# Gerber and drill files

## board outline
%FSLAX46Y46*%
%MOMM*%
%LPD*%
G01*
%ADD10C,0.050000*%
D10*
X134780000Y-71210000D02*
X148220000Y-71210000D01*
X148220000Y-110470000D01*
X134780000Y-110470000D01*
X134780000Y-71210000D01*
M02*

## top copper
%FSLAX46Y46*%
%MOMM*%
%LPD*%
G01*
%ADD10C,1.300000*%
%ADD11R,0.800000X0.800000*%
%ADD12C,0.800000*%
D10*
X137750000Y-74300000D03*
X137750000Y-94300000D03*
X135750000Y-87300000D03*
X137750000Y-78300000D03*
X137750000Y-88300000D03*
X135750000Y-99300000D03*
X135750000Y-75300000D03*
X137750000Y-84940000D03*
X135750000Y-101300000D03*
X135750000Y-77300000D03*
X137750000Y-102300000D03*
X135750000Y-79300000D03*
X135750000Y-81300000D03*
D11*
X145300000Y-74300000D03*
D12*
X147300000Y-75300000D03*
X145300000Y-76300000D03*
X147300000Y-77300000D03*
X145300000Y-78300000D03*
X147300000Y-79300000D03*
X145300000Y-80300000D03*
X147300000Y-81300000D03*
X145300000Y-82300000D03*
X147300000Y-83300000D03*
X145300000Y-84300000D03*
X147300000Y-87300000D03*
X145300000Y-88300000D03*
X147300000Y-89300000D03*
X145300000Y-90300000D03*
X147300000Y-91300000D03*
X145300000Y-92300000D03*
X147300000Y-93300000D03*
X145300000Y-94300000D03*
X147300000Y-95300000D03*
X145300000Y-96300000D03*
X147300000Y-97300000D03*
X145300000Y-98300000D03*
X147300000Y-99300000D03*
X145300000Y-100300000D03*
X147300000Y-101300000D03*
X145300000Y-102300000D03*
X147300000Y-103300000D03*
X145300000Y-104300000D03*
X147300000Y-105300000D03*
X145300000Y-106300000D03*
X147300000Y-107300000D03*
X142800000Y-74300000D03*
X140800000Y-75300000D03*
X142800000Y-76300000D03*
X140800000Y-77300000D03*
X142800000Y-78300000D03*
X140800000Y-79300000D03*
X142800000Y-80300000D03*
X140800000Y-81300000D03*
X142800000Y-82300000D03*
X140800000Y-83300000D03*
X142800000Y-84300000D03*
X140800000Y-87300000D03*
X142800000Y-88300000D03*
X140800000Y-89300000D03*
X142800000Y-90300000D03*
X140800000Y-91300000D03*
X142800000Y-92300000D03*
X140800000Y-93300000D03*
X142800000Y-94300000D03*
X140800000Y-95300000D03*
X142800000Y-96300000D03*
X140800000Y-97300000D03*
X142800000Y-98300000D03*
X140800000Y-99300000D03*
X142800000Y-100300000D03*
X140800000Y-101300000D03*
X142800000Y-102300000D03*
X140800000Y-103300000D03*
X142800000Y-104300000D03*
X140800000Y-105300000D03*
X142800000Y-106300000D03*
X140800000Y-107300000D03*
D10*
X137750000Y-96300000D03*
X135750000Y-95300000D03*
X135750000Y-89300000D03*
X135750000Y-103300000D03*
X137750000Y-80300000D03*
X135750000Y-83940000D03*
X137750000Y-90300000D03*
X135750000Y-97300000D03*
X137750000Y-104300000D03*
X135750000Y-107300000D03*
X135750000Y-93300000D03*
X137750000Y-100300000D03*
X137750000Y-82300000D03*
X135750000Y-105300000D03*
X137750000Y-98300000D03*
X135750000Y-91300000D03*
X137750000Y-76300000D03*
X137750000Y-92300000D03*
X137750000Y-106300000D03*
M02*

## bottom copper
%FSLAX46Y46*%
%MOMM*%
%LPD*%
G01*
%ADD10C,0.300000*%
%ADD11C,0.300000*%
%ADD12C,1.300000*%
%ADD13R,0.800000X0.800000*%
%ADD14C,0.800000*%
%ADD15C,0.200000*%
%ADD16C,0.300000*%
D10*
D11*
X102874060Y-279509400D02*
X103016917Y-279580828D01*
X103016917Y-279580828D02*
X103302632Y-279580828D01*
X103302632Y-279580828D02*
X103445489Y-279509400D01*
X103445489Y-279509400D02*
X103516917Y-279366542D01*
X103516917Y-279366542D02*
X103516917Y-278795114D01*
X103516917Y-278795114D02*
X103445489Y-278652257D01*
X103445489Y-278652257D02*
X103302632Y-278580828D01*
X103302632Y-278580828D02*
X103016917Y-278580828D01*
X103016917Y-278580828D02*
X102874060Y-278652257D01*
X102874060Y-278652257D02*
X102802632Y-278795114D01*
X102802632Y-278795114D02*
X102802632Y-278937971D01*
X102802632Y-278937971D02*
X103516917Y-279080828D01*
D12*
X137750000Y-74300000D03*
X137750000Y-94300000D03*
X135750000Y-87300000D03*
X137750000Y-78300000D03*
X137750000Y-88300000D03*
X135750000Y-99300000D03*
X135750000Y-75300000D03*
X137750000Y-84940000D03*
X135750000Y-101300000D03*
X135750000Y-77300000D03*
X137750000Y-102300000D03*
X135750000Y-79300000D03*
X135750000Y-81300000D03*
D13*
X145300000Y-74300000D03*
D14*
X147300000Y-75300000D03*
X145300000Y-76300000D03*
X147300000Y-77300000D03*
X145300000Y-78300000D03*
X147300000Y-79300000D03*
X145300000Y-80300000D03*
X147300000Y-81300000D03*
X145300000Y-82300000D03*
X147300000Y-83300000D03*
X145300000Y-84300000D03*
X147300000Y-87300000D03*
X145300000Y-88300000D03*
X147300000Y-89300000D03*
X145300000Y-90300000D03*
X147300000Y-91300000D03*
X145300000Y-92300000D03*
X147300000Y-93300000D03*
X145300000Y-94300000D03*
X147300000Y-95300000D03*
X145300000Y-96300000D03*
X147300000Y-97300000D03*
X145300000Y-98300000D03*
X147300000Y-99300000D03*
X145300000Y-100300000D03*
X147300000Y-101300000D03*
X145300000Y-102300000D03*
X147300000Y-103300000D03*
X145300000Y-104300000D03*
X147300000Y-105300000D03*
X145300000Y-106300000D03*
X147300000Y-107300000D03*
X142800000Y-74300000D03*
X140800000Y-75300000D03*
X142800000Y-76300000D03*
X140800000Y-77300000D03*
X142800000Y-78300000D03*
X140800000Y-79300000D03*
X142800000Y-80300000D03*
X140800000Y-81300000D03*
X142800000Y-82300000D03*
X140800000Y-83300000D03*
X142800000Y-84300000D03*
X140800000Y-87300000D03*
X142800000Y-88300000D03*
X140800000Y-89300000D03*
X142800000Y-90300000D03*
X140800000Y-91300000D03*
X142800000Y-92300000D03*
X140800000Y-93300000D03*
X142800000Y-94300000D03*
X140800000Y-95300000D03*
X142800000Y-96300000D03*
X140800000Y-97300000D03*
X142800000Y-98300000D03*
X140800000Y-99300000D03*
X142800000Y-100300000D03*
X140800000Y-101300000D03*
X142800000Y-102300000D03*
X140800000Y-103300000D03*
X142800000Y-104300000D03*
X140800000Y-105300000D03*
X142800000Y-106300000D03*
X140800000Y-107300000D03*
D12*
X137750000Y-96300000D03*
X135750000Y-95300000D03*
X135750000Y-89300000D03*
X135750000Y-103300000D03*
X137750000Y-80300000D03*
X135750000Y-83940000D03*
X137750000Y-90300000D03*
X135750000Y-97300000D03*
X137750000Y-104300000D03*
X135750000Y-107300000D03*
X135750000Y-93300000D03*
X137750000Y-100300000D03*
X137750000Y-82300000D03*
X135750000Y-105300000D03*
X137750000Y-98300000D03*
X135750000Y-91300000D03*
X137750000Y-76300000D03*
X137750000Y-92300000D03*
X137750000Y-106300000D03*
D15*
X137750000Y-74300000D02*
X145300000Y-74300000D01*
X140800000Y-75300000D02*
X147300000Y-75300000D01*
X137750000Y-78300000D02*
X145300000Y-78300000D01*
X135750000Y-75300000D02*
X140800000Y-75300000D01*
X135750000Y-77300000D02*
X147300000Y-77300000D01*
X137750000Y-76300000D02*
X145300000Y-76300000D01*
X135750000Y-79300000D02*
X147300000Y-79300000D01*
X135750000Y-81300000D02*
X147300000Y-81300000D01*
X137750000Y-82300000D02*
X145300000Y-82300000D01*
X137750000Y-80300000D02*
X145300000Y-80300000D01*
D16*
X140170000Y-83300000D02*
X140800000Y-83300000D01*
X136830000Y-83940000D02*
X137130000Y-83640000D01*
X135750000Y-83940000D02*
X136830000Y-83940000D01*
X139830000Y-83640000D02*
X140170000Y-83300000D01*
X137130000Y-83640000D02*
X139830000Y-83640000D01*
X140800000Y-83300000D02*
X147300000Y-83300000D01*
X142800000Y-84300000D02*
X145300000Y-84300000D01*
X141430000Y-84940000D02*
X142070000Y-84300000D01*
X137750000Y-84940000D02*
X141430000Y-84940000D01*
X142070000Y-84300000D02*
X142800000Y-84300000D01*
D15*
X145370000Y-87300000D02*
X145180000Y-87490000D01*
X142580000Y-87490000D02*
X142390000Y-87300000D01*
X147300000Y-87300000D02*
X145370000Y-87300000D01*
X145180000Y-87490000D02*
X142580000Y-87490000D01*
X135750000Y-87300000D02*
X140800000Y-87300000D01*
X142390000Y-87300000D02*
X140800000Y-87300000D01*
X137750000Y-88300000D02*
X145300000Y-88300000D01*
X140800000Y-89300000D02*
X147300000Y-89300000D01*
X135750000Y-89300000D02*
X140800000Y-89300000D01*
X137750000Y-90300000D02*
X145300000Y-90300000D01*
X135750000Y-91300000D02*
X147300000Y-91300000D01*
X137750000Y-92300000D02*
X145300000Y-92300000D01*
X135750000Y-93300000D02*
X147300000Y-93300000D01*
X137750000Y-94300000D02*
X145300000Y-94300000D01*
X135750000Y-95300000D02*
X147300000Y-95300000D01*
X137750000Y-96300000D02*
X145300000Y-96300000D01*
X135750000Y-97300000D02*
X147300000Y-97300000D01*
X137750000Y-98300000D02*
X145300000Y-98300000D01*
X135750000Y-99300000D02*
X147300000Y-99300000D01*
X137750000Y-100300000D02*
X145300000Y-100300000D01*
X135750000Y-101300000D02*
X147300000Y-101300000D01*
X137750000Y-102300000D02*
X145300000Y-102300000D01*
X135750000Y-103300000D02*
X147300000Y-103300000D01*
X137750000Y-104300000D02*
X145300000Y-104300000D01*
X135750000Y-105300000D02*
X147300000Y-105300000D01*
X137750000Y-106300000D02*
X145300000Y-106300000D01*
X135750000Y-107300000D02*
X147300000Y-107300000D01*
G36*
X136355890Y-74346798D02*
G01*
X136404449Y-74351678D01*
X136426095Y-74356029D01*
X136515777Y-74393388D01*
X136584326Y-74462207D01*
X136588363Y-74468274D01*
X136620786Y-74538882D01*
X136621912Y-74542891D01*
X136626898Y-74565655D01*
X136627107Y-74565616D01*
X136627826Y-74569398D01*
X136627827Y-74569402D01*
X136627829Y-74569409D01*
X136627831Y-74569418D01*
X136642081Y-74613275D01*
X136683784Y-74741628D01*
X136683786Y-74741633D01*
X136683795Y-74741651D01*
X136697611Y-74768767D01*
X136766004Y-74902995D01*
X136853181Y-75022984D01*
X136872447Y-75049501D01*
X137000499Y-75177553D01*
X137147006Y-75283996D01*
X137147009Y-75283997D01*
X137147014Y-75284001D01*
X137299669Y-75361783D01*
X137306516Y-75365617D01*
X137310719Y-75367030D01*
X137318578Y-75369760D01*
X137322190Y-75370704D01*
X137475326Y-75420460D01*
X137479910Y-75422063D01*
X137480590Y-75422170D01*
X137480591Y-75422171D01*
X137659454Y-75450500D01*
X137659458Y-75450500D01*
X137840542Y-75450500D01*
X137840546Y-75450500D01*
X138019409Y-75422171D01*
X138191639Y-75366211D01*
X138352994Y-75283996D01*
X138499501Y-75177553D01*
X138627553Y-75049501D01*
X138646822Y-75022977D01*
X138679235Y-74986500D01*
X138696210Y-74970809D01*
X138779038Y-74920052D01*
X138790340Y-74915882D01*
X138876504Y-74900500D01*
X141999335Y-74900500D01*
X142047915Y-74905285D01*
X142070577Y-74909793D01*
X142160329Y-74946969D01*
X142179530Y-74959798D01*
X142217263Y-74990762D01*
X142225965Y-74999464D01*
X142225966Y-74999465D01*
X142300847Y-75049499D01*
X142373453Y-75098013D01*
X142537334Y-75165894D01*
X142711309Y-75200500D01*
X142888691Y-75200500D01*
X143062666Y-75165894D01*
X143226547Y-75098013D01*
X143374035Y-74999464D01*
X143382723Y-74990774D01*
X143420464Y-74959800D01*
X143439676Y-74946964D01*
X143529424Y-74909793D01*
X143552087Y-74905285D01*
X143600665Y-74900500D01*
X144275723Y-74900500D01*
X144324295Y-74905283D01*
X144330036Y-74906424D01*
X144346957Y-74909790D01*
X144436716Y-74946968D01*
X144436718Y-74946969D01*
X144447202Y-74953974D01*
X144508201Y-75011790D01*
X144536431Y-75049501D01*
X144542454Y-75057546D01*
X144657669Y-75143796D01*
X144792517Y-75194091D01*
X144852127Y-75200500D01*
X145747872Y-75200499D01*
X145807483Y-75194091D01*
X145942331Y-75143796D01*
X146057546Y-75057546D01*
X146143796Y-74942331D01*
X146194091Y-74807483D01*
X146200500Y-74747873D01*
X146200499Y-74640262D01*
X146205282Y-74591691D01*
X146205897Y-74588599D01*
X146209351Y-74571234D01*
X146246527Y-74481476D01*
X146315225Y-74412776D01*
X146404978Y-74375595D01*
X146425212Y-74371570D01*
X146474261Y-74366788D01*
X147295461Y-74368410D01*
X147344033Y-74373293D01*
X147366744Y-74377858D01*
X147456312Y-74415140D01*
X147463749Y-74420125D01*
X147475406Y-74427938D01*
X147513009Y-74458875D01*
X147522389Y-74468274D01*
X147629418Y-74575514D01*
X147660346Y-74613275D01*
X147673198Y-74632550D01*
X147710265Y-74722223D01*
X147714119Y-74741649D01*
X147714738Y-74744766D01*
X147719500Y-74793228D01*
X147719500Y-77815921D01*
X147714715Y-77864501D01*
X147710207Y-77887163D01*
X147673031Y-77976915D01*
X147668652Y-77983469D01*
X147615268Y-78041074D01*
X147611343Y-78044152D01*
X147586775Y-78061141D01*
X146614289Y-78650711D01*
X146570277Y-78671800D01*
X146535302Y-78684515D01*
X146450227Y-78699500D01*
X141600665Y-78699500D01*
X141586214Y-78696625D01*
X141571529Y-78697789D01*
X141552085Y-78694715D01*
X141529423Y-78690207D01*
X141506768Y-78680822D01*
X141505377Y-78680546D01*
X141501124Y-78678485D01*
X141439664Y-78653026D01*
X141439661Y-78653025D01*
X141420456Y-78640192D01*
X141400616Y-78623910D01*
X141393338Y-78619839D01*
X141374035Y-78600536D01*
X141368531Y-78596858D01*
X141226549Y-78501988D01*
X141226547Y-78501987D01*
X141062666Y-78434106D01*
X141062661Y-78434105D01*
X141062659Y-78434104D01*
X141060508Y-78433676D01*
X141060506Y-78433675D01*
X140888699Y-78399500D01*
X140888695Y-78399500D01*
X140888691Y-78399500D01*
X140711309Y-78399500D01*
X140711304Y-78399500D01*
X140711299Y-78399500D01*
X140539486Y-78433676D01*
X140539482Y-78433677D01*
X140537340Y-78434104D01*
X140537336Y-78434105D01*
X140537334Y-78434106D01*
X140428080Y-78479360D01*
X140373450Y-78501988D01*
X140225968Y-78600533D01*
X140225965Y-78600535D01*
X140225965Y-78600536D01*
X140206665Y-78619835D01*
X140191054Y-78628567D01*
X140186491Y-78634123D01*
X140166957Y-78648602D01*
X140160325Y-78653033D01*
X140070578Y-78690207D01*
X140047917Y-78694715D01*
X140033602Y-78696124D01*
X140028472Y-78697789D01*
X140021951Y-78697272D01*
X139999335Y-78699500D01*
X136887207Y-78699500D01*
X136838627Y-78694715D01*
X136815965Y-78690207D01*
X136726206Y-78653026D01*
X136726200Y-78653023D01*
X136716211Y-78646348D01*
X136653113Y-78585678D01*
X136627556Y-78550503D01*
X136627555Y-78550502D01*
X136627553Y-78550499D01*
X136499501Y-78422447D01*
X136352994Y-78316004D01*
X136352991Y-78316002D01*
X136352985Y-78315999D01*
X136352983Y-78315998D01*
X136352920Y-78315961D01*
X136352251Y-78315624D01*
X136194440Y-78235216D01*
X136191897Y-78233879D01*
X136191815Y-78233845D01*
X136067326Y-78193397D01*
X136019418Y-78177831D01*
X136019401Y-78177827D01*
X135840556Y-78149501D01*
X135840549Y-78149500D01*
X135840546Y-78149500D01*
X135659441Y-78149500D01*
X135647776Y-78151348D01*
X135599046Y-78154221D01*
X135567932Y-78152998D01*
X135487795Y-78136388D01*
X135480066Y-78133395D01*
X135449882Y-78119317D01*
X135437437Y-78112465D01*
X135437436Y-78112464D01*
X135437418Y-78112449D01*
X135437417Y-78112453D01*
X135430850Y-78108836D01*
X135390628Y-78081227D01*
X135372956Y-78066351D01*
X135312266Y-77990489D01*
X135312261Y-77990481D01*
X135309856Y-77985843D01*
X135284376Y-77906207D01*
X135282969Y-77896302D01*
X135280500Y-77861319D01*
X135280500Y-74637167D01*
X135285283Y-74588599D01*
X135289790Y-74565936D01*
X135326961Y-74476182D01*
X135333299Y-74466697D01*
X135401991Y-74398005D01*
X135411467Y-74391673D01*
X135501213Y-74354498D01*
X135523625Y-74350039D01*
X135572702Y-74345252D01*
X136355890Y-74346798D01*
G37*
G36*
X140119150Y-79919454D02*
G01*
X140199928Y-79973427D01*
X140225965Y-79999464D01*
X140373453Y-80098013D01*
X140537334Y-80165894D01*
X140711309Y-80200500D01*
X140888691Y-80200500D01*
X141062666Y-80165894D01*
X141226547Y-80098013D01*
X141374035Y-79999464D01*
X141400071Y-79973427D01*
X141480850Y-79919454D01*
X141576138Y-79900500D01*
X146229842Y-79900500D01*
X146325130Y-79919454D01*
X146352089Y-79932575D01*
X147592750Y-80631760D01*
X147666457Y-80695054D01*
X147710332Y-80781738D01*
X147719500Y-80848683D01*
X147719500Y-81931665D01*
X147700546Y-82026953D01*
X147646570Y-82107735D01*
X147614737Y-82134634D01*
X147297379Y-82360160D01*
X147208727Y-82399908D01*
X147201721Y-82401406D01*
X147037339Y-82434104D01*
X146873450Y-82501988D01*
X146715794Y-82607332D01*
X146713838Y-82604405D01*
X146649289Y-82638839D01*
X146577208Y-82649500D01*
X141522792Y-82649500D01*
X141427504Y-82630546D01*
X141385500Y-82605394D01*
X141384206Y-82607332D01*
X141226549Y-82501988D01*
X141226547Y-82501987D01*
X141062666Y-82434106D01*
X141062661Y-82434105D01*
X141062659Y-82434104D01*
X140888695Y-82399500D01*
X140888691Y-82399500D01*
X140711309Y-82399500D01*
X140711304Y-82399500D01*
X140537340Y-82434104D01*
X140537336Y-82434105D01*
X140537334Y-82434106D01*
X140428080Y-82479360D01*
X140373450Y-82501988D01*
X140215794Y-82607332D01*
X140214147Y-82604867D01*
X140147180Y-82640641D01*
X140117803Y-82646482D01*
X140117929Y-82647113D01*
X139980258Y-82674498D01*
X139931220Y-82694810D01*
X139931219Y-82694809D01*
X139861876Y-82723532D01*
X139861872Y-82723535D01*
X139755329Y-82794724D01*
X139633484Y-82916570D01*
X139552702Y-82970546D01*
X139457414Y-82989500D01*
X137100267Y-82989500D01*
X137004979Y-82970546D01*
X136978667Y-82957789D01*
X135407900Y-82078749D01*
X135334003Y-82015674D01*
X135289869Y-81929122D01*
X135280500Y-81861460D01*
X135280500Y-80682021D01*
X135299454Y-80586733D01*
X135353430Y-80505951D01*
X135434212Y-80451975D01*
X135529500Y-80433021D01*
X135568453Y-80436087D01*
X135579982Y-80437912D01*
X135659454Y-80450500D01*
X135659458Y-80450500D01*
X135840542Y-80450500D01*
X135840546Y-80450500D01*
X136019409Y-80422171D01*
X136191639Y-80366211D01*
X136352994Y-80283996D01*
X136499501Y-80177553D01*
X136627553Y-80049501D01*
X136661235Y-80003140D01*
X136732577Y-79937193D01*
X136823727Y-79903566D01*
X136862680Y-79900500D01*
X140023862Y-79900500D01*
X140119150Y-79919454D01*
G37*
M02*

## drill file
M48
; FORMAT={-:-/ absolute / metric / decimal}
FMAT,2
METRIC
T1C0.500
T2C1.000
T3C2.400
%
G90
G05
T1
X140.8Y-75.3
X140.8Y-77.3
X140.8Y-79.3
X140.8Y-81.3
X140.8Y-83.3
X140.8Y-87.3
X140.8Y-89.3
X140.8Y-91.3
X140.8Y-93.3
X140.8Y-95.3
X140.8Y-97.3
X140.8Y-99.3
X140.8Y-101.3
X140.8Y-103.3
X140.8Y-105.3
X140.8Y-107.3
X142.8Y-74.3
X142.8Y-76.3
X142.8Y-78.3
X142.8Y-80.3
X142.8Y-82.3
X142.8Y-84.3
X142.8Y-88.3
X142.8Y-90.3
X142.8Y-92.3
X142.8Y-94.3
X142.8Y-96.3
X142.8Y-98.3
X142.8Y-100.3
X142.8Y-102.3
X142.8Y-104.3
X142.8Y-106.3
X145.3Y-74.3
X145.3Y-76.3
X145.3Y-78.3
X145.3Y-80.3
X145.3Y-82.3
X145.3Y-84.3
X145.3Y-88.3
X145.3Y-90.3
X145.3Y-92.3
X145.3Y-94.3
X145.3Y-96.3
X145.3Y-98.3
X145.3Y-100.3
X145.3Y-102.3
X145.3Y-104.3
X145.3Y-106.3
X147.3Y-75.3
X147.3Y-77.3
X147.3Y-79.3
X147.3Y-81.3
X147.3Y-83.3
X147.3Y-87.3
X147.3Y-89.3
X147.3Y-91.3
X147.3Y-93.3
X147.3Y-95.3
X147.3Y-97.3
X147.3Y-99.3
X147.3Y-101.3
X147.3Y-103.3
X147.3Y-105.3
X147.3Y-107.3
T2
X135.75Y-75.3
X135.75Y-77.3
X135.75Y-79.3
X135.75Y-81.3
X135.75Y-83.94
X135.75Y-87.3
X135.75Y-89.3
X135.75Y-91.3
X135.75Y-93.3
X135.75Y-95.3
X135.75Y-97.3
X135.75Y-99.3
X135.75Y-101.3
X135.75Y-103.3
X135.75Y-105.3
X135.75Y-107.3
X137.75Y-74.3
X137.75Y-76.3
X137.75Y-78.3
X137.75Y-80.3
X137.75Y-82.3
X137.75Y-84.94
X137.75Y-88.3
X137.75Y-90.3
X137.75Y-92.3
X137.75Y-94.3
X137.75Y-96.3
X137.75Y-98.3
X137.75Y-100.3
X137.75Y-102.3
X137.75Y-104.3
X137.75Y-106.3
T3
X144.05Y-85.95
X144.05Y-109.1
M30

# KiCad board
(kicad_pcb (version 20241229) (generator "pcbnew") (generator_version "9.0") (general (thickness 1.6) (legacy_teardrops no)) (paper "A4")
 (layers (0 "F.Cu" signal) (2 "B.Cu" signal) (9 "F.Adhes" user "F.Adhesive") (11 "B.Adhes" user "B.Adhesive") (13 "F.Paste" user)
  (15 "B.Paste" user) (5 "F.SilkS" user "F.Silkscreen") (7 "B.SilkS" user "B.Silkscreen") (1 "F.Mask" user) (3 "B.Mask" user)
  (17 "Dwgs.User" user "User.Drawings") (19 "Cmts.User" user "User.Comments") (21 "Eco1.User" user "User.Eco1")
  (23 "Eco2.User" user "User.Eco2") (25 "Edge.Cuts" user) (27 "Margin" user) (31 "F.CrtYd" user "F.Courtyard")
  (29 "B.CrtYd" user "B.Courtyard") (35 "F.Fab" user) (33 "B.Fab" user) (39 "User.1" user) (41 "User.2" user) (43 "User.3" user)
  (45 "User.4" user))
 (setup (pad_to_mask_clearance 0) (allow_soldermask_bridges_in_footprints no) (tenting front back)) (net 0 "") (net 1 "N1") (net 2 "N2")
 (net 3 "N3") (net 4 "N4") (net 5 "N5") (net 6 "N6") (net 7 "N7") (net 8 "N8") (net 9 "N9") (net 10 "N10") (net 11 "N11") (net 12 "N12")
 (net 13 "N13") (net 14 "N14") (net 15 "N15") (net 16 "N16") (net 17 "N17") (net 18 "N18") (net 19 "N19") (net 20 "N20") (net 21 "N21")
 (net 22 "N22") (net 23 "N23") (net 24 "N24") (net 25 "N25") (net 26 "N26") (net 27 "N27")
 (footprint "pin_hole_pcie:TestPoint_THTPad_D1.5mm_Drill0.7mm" (layer "F.Cu") (at 137.75 74.3 180)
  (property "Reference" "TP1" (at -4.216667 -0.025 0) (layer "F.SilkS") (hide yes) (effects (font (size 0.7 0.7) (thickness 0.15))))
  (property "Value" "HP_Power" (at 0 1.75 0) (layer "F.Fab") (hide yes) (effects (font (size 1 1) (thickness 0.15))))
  (pad "1" thru_hole circle (at 0 0 180) (size 1.3 1.3) (drill 1) (layers "*.Cu" "*.Mask") (remove_unused_layers no) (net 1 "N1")))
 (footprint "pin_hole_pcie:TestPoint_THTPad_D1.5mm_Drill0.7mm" (layer "F.Cu") (at 137.75 94.3 180)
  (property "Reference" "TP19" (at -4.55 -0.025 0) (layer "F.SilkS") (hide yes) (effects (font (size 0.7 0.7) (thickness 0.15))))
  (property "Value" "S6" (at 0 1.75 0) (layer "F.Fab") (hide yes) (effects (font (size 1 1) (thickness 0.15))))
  (pad "1" thru_hole circle (at 0 0 180) (size 1.3 1.5) (drill 1) (layers "*.Cu" "*.Mask") (remove_unused_layers no) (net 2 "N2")))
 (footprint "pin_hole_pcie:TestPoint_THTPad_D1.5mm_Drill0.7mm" (layer "F.Cu") (at 135.75 87.3 180)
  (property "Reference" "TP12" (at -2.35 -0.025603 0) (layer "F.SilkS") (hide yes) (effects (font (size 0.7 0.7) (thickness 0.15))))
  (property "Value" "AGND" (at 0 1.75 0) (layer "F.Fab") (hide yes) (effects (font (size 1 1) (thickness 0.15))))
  (pad "1" thru_hole circle (at 0 0 180) (size 1.3 1.5) (drill 1) (layers "*.Cu" "*.Mask") (remove_unused_layers no) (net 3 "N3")))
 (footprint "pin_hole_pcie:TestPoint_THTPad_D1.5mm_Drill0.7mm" (layer "F.Cu") (at 137.75 78.3 180)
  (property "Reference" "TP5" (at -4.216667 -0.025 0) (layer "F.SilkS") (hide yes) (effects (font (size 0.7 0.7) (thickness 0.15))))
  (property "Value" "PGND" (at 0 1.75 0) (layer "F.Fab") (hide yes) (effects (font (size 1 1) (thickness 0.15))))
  (pad "1" thru_hole circle (at 0 0 180) (size 1.3 1.5) (drill 1) (layers "*.Cu" "*.Mask") (remove_unused_layers no) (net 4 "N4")))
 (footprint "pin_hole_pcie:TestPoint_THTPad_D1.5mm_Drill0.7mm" (layer "F.Cu") (at 137.75 88.3 180)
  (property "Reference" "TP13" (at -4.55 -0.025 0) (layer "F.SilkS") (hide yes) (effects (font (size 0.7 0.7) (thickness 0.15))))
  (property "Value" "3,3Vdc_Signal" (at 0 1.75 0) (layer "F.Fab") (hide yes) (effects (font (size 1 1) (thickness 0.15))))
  (pad "1" thru_hole circle (at 0 0 180) (size 1.3 1.5) (drill 1) (layers "*.Cu" "*.Mask") (remove_unused_layers no) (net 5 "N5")))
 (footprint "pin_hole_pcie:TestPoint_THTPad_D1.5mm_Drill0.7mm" (layer "F.Cu") (at 135.75 99.3 180)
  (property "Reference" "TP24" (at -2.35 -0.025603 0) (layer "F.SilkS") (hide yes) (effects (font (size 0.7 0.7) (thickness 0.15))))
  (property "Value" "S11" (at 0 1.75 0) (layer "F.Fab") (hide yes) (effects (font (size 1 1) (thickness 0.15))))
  (pad "1" thru_hole circle (at 0 0 180) (size 1.3 1.5) (drill 1) (layers "*.Cu" "*.Mask") (remove_unused_layers no) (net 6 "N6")))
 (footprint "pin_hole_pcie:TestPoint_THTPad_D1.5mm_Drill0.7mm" (layer "F.Cu") (at 135.75 75.3 180)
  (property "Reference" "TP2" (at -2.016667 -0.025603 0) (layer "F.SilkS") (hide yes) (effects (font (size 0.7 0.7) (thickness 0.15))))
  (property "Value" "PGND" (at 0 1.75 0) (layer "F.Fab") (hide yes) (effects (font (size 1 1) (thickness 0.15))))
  (pad "1" thru_hole circle (at 0 0 180) (size 1.3 1.5) (drill 1) (layers "*.Cu" "*.Mask") (remove_unused_layers no) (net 4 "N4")))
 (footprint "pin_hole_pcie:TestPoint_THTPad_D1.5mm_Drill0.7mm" (layer "F.Cu") (at 137.75 84.94 180)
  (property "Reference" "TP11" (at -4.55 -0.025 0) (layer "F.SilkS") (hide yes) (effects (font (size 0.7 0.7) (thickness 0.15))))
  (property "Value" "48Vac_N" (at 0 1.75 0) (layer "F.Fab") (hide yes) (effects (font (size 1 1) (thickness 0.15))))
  (pad "1" thru_hole circle (at 0 0 180) (size 1.3 1.5) (drill 1) (layers "*.Cu" "*.Mask") (remove_unused_layers no) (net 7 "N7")))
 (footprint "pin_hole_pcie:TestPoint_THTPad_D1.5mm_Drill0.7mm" (layer "F.Cu") (at 135.75 101.3 180)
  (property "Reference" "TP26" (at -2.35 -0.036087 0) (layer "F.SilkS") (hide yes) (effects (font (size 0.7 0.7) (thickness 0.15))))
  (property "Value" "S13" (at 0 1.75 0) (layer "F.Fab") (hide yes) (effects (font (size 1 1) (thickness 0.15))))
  (pad "1" thru_hole circle (at 0 0 180) (size 1.3 1.5) (drill 1) (layers "*.Cu" "*.Mask") (remove_unused_layers no) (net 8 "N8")))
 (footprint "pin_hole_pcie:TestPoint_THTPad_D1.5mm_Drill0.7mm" (layer "F.Cu") (at 135.75 77.3 180)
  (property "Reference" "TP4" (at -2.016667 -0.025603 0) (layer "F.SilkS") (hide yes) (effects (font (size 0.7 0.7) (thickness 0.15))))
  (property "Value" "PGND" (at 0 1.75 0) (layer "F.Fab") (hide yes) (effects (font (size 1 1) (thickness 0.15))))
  (pad "1" thru_hole circle (at 0 0 180) (size 1.3 1.5) (drill 1) (layers "*.Cu" "*.Mask") (remove_unused_layers no) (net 4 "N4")))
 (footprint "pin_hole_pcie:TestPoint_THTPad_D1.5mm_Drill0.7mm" (layer "F.Cu") (at 137.75 102.3 180)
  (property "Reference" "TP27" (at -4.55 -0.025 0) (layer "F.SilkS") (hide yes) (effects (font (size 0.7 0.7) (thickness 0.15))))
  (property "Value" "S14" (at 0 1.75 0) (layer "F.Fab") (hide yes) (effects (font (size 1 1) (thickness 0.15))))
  (pad "1" thru_hole circle (at 0 0 180) (size 1.3 1.5) (drill 1) (layers "*.Cu" "*.Mask") (remove_unused_layers no) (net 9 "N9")))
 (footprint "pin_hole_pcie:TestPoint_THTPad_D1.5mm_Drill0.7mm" (layer "F.Cu") (at 135.75 79.3 180)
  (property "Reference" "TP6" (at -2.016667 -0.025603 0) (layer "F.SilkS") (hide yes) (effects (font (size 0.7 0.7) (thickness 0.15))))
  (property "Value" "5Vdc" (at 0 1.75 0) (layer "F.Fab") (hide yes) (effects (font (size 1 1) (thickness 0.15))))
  (pad "1" thru_hole circle (at 0 0 180) (size 1.3 1.5) (drill 1) (layers "*.Cu" "*.Mask") (remove_unused_layers no) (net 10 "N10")))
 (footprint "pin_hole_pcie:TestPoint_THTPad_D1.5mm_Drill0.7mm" (layer "F.Cu") (at 135.75 81.3 180)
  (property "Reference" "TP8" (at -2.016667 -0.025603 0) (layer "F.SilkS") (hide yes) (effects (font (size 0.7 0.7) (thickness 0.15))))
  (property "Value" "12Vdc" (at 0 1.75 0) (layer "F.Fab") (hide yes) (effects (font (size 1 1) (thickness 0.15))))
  (pad "1" thru_hole circle (at 0 0 180) (size 1.3 1.5) (drill 1) (layers "*.Cu" "*.Mask") (remove_unused_layers no) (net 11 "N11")))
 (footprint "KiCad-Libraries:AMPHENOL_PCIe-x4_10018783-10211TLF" (layer "F.Cu") (at 144.05 85.95 -90)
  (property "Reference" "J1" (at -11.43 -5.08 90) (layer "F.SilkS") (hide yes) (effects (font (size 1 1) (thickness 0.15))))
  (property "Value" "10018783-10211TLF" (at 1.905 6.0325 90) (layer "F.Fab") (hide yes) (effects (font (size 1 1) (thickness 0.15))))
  (pad "" np_thru_hole circle (at 0 0 270) (size 2.4 2.4) (drill 2.4) (layers "*.Cu" "*.Mask"))
  (pad "" np_thru_hole circle (at 23.15 0 270) (size 2.4 2.4) (drill 2.4) (layers "*.Cu" "*.Mask"))
  (pad "A1" thru_hole rect (at -11.65 -1.25 270) (size 0.8 0.8) (drill 0.5) (layers "*.Cu" "*.Mask") (remove_unused_layers no) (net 1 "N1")
   (solder_mask_margin 0.102))
  (pad "A2" thru_hole circle (at -10.65 -3.25 270) (size 0.8 1.288) (drill 0.5) (layers "*.Cu" "*.Mask") (remove_unused_layers no)
   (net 4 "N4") (solder_mask_margin 0.102))
  (pad "A3" thru_hole circle (at -9.65 -1.25 270) (size 0.8 1.288) (drill 0.5) (layers "*.Cu" "*.Mask") (remove_unused_layers no)
   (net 4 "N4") (solder_mask_margin 0.102))
  (pad "A4" thru_hole circle (at -8.65 -3.25 270) (size 0.8 1.288) (drill 0.5) (layers "*.Cu" "*.Mask") (remove_unused_layers no)
   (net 4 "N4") (solder_mask_margin 0.102))
  (pad "A5" thru_hole circle (at -7.65 -1.25 270) (size 0.8 1.288) (drill 0.5) (layers "*.Cu" "*.Mask") (remove_unused_layers no)
   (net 4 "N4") (solder_mask_margin 0.102))
  (pad "A6" thru_hole circle (at -6.65 -3.25 270) (size 0.8 1.288) (drill 0.5) (layers "*.Cu" "*.Mask") (remove_unused_layers no)
   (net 10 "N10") (solder_mask_margin 0.102))
  (pad "A7" thru_hole circle (at -5.65 -1.25 270) (size 0.8 1.288) (drill 0.5) (layers "*.Cu" "*.Mask") (remove_unused_layers no)
   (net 11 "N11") (solder_mask_margin 0.102))
  (pad "A8" thru_hole circle (at -4.65 -3.25 270) (size 0.8 1.288) (drill 0.5) (layers "*.Cu" "*.Mask") (remove_unused_layers no)
   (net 11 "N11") (solder_mask_margin 0.102))
  (pad "A9" thru_hole circle (at -3.65 -1.25 270) (size 0.8 1.288) (drill 0.5) (layers "*.Cu" "*.Mask") (remove_unused_layers no)
   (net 11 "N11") (solder_mask_margin 0.102))
  (pad "A10" thru_hole circle (at -2.65 -3.25 270) (size 0.8 1.288) (drill 0.5) (layers "*.Cu" "*.Mask") (remove_unused_layers no)
   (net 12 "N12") (solder_mask_margin 0.102))
  (pad "A11" thru_hole circle (at -1.65 -1.25 270) (size 0.8 1.288) (drill 0.5) (layers "*.Cu" "*.Mask") (remove_unused_layers no)
   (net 7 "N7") (solder_mask_margin 0.102))
  (pad "A12" thru_hole circle (at 1.35 -3.25 270) (size 0.8 1.288) (drill 0.5) (layers "*.Cu" "*.Mask") (remove_unused_layers no)
   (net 3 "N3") (solder_mask_margin 0.102))
  (pad "A13" thru_hole circle (at 2.35 -1.25 270) (size 0.8 1.288) (drill 0.5) (layers "*.Cu" "*.Mask") (remove_unused_layers no)
   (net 5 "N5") (solder_mask_margin 0.102))
  (pad "A14" thru_hole circle (at 3.35 -3.25 270) (size 0.8 1.288) (drill 0.5) (layers "*.Cu" "*.Mask") (remove_unused_layers no)
   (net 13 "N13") (solder_mask_margin 0.102))
  (pad "A15" thru_hole circle (at 4.35 -1.25 270) (size 0.8 1.288) (drill 0.5) (layers "*.Cu" "*.Mask") (remove_unused_layers no)
   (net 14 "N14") (solder_mask_margin 0.102))
  (pad "A16" thru_hole circle (at 5.35 -3.25 270) (size 0.8 1.288) (drill 0.5) (layers "*.Cu" "*.Mask") (remove_unused_layers no)
   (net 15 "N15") (solder_mask_margin 0.102))
  (pad "A17" thru_hole circle (at 6.35 -1.25 270) (size 0.8 1.288) (drill 0.5) (layers "*.Cu" "*.Mask") (remove_unused_layers no)
   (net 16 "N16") (solder_mask_margin 0.102))
  (pad "A18" thru_hole circle (at 7.35 -3.25 270) (size 0.8 1.288) (drill 0.5) (layers "*.Cu" "*.Mask") (remove_unused_layers no)
   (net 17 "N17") (solder_mask_margin 0.102))
  (pad "A19" thru_hole circle (at 8.35 -1.25 270) (size 0.8 1.288) (drill 0.5) (layers "*.Cu" "*.Mask") (remove_unused_layers no)
   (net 2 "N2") (solder_mask_margin 0.102))
  (pad "A20" thru_hole circle (at 9.35 -3.25 270) (size 0.8 1.288) (drill 0.5) (layers "*.Cu" "*.Mask") (remove_unused_layers no)
   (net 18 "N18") (solder_mask_margin 0.102))
  (pad "A21" thru_hole circle (at 10.35 -1.25 270) (size 0.8 1.288) (drill 0.5) (layers "*.Cu" "*.Mask") (remove_unused_layers no)
   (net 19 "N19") (solder_mask_margin 0.102))
  (pad "A22" thru_hole circle (at 11.35 -3.25 270) (size 0.8 1.288) (drill 0.5) (layers "*.Cu" "*.Mask") (remove_unused_layers no)
   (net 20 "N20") (solder_mask_margin 0.102))
  (pad "A23" thru_hole circle (at 12.35 -1.25 270) (size 0.8 1.288) (drill 0.5) (layers "*.Cu" "*.Mask") (remove_unused_layers no)
   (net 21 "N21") (solder_mask_margin 0.102))
  (pad "A24" thru_hole circle (at 13.35 -3.25 270) (size 0.8 1.288) (drill 0.5) (layers "*.Cu" "*.Mask") (remove_unused_layers no)
   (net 6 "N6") (solder_mask_margin 0.102))
  (pad "A25" thru_hole circle (at 14.35 -1.25 270) (size 0.8 1.288) (drill 0.5) (layers "*.Cu" "*.Mask") (remove_unused_layers no)
   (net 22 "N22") (solder_mask_margin 0.102))
  (pad "A26" thru_hole circle (at 15.35 -3.25 270) (size 0.8 1.288) (drill 0.5) (layers "*.Cu" "*.Mask") (remove_unused_layers no)
   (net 8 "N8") (solder_mask_margin 0.102))
  (pad "A27" thru_hole circle (at 16.35 -1.25 270) (size 0.8 1.288) (drill 0.5) (layers "*.Cu" "*.Mask") (remove_unused_layers no)
   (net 9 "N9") (solder_mask_margin 0.102))
  (pad "A28" thru_hole circle (at 17.35 -3.25 270) (size 0.8 1.288) (drill 0.5) (layers "*.Cu" "*.Mask") (remove_unused_layers no)
   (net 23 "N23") (solder_mask_margin 0.102))
  (pad "A29" thru_hole circle (at 18.35 -1.25 270) (size 0.8 1.288) (drill 0.5) (layers "*.Cu" "*.Mask") (remove_unused_layers no)
   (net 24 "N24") (solder_mask_margin 0.102))
  (pad "A30" thru_hole circle (at 19.35 -3.25 270) (size 0.8 1.288) (drill 0.5) (layers "*.Cu" "*.Mask") (remove_unused_layers no)
   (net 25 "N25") (solder_mask_margin 0.102))
  (pad "A31" thru_hole circle (at 20.35 -1.25 270) (size 0.8 1.288) (drill 0.5) (layers "*.Cu" "*.Mask") (remove_unused_layers no)
   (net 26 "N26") (solder_mask_margin 0.102))
  (pad "A32" thru_hole circle (at 21.35 -3.25 270) (size 0.8 1.288) (drill 0.5) (layers "*.Cu" "*.Mask") (remove_unused_layers no)
   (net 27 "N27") (solder_mask_margin 0.102))
  (pad "B1" thru_hole circle (at -11.65 1.25 270) (size 0.8 1.288) (drill 0.5) (layers "*.Cu" "*.Mask") (remove_unused_layers no)
   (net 1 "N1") (solder_mask_margin 0.102))
  (pad "B2" thru_hole circle (at -10.65 3.25 270) (size 0.8 1.288) (drill 0.5) (layers "*.Cu" "*.Mask") (remove_unused_layers no)
   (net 4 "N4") (solder_mask_margin 0.102))
  (pad "B3" thru_hole circle (at -9.65 1.25 270) (size 0.8 1.288) (drill 0.5) (layers "*.Cu" "*.Mask") (remove_unused_layers no)
   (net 4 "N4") (solder_mask_margin 0.102))
  (pad "B4" thru_hole circle (at -8.65 3.25 270) (size 0.8 1.288) (drill 0.5) (layers "*.Cu" "*.Mask") (remove_unused_layers no)
   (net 4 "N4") (solder_mask_margin 0.102))
  (pad "B5" thru_hole circle (at -7.65 1.25 270) (size 0.8 1.288) (drill 0.5) (layers "*.Cu" "*.Mask") (remove_unused_layers no)
   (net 4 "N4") (solder_mask_margin 0.102))
  (pad "B6" thru_hole circle (at -6.65 3.25 270) (size 0.8 1.288) (drill 0.5) (layers "*.Cu" "*.Mask") (remove_unused_layers no)
   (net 10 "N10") (solder_mask_margin 0.102))
  (pad "B7" thru_hole circle (at -5.65 1.25 270) (size 0.8 1.288) (drill 0.5) (layers "*.Cu" "*.Mask") (remove_unused_layers no)
   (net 11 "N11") (solder_mask_margin 0.102))
  (pad "B8" thru_hole circle (at -4.65 3.25 270) (size 0.8 1.288) (drill 0.5) (layers "*.Cu" "*.Mask") (remove_unused_layers no)
   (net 11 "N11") (solder_mask_margin 0.102))
  (pad "B9" thru_hole circle (at -3.65 1.25 270) (size 0.8 1.288) (drill 0.5) (layers "*.Cu" "*.Mask") (remove_unused_layers no)
   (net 11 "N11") (solder_mask_margin 0.102))
  (pad "B10" thru_hole circle (at -2.65 3.25 270) (size 0.8 1.288) (drill 0.5) (layers "*.Cu" "*.Mask") (remove_unused_layers no)
   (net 12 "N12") (solder_mask_margin 0.102))
  (pad "B11" thru_hole circle (at -1.65 1.25 270) (size 0.8 1.288) (drill 0.5) (layers "*.Cu" "*.Mask") (remove_unused_layers no)
   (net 7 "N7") (solder_mask_margin 0.102))
  (pad "B12" thru_hole circle (at 1.35 3.25 270) (size 0.8 1.288) (drill 0.5) (layers "*.Cu" "*.Mask") (remove_unused_layers no)
   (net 3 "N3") (solder_mask_margin 0.102))
  (pad "B13" thru_hole circle (at 2.35 1.25 270) (size 0.8 1.288) (drill 0.5) (layers "*.Cu" "*.Mask") (remove_unused_layers no)
   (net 5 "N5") (solder_mask_margin 0.102))
  (pad "B14" thru_hole circle (at 3.35 3.25 270) (size 0.8 1.288) (drill 0.5) (layers "*.Cu" "*.Mask") (remove_unused_layers no)
   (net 13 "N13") (solder_mask_margin 0.102))
  (pad "B15" thru_hole circle (at 4.35 1.25 270) (size 0.8 1.288) (drill 0.5) (layers "*.Cu" "*.Mask") (remove_unused_layers no)
   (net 14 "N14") (solder_mask_margin 0.102))
  (pad "B16" thru_hole circle (at 5.35 3.25 270) (size 0.8 1.288) (drill 0.5) (layers "*.Cu" "*.Mask") (remove_unused_layers no)
   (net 15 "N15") (solder_mask_margin 0.102))
  (pad "B17" thru_hole circle (at 6.35 1.25 270) (size 0.8 1.288) (drill 0.5) (layers "*.Cu" "*.Mask") (remove_unused_layers no)
   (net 16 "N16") (solder_mask_margin 0.102))
  (pad "B18" thru_hole circle (at 7.35 3.25 270) (size 0.8 1.288) (drill 0.5) (layers "*.Cu" "*.Mask") (remove_unused_layers no)
   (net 17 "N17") (solder_mask_margin 0.102))
  (pad "B19" thru_hole circle (at 8.35 1.25 270) (size 0.8 1.288) (drill 0.5) (layers "*.Cu" "*.Mask") (remove_unused_layers no)
   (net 2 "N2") (solder_mask_margin 0.102))
  (pad "B20" thru_hole circle (at 9.35 3.25 270) (size 0.8 1.288) (drill 0.5) (layers "*.Cu" "*.Mask") (remove_unused_layers no)
   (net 18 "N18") (solder_mask_margin 0.102))
  (pad "B21" thru_hole circle (at 10.35 1.25 270) (size 0.8 1.288) (drill 0.5) (layers "*.Cu" "*.Mask") (remove_unused_layers no)
   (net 19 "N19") (solder_mask_margin 0.102))
  (pad "B22" thru_hole circle (at 11.35 3.25 270) (size 0.8 1.288) (drill 0.5) (layers "*.Cu" "*.Mask") (remove_unused_layers no)
   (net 20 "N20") (solder_mask_margin 0.102))
  (pad "B23" thru_hole circle (at 12.35 1.25 270) (size 0.8 1.288) (drill 0.5) (layers "*.Cu" "*.Mask") (remove_unused_layers no)
   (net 21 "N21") (solder_mask_margin 0.102))
  (pad "B24" thru_hole circle (at 13.35 3.25 270) (size 0.8 1.288) (drill 0.5) (layers "*.Cu" "*.Mask") (remove_unused_layers no)
   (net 6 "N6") (solder_mask_margin 0.102))
  (pad "B25" thru_hole circle (at 14.35 1.25 270) (size 0.8 1.288) (drill 0.5) (layers "*.Cu" "*.Mask") (remove_unused_layers no)
   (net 22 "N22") (solder_mask_margin 0.102))
  (pad "B26" thru_hole circle (at 15.35 3.25 270) (size 0.8 1.288) (drill 0.5) (layers "*.Cu" "*.Mask") (remove_unused_layers no)
   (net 8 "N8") (solder_mask_margin 0.102))
  (pad "B27" thru_hole circle (at 16.35 1.25 270) (size 0.8 1.288) (drill 0.5) (layers "*.Cu" "*.Mask") (remove_unused_layers no)
   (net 9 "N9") (solder_mask_margin 0.102))
  (pad "B28" thru_hole circle (at 17.35 3.25 270) (size 0.8 1.288) (drill 0.5) (layers "*.Cu" "*.Mask") (remove_unused_layers no)
   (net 23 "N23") (solder_mask_margin 0.102))
  (pad "B29" thru_hole circle (at 18.35 1.25 270) (size 0.8 1.288) (drill 0.5) (layers "*.Cu" "*.Mask") (remove_unused_layers no)
   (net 24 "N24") (solder_mask_margin 0.102))
  (pad "B30" thru_hole circle (at 19.35 3.25 270) (size 0.8 1.288) (drill 0.5) (layers "*.Cu" "*.Mask") (remove_unused_layers no)
   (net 25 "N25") (solder_mask_margin 0.102))
  (pad "B31" thru_hole circle (at 20.35 1.25 270) (size 0.8 1.288) (drill 0.5) (layers "*.Cu" "*.Mask") (remove_unused_layers no)
   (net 26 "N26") (solder_mask_margin 0.102))
  (pad "B32" thru_hole circle (at 21.35 3.25 270) (size 0.8 1.288) (drill 0.5) (layers "*.Cu" "*.Mask") (remove_unused_layers no)
   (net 27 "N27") (solder_mask_margin 0.102)))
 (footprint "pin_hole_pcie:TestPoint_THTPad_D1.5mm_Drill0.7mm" (layer "F.Cu") (at 137.75 96.3 180)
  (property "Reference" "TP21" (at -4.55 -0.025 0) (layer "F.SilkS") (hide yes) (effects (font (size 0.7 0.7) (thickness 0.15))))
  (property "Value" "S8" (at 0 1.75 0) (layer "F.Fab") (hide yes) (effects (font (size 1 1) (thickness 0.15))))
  (pad "1" thru_hole circle (at 0 0 180) (size 1.3 1.5) (drill 1) (layers "*.Cu" "*.Mask") (remove_unused_layers no) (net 19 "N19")))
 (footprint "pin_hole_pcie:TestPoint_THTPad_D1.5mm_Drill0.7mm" (layer "F.Cu") (at 135.75 95.3 180)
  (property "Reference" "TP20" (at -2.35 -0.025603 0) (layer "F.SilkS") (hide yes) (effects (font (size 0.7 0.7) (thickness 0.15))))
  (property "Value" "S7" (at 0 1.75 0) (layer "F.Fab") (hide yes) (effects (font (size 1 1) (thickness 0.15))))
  (pad "1" thru_hole circle (at 0 0 180) (size 1.3 1.5) (drill 1) (layers "*.Cu" "*.Mask") (remove_unused_layers no) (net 18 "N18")))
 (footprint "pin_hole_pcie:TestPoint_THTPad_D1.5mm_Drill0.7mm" (layer "F.Cu") (at 135.75 89.3 180)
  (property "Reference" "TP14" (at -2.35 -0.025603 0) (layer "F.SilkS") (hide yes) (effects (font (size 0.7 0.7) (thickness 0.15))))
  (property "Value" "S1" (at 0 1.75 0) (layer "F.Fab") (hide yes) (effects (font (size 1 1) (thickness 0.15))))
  (pad "1" thru_hole circle (at 0 0 180) (size 1.3 1.5) (drill 1) (layers "*.Cu" "*.Mask") (remove_unused_layers no) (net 13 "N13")))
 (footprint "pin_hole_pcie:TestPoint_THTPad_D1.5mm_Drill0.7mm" (layer "F.Cu") (at 135.75 103.3 180)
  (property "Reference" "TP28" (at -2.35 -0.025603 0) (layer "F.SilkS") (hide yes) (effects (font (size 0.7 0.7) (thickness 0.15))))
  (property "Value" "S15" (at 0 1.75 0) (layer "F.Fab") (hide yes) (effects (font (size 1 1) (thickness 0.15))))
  (pad "1" thru_hole circle (at 0 0 180) (size 1.3 1.5) (drill 1) (layers "*.Cu" "*.Mask") (remove_unused_layers no) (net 23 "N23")))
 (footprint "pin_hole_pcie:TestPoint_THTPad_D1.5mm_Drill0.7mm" (layer "F.Cu") (at 137.75 80.3 180)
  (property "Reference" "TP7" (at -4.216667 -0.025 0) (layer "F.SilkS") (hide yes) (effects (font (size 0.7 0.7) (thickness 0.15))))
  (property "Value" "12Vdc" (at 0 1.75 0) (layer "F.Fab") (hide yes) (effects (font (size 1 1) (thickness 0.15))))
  (pad "1" thru_hole circle (at 0 0 180) (size 1.3 1.5) (drill 1) (layers "*.Cu" "*.Mask") (remove_unused_layers no) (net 11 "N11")))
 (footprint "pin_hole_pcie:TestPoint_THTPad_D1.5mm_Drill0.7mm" (layer "F.Cu") (at 135.75 83.94 180)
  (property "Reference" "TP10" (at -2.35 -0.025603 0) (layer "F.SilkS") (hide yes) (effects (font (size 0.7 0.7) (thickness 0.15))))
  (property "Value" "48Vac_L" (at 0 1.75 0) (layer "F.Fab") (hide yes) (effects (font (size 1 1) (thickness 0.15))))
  (pad "1" thru_hole circle (at 0 0 180) (size 1.3 1.5) (drill 1) (layers "*.Cu" "*.Mask") (remove_unused_layers no) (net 12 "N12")))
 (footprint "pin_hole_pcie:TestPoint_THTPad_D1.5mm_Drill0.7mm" (layer "F.Cu") (at 137.75 90.3 180)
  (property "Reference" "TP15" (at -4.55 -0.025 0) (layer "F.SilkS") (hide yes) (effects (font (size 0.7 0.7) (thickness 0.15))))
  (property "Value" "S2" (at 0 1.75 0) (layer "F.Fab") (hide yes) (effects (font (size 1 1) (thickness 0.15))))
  (pad "1" thru_hole circle (at 0 0 180) (size 1.3 1.5) (drill 1) (layers "*.Cu" "*.Mask") (remove_unused_layers no) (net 14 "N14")))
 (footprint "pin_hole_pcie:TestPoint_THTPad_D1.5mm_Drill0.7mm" (layer "F.Cu") (at 135.75 97.3 180)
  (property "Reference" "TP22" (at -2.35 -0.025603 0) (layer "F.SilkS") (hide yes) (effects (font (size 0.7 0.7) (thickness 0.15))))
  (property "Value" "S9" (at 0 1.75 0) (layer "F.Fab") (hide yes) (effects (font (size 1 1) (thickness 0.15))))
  (pad "1" thru_hole circle (at 0 0 180) (size 1.3 1.5) (drill 1) (layers "*.Cu" "*.Mask") (remove_unused_layers no) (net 20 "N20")))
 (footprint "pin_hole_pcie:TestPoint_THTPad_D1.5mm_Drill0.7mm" (layer "F.Cu") (at 137.75 104.3 180)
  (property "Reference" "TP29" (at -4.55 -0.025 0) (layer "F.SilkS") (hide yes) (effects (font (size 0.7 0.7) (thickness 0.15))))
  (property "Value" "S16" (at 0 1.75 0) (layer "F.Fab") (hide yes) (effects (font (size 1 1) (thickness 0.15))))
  (pad "1" thru_hole circle (at 0 0 180) (size 1.3 1.5) (drill 1) (layers "*.Cu" "*.Mask") (remove_unused_layers no) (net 24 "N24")))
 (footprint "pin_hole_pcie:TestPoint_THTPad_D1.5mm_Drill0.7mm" (layer "F.Cu") (at 135.75 107.3 180)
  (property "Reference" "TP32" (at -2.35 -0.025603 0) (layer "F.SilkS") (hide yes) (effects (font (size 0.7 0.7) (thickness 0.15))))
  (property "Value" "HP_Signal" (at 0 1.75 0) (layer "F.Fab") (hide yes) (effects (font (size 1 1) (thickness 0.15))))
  (pad "1" thru_hole circle (at 0 0 180) (size 1.3 1.5) (drill 1) (layers "*.Cu" "*.Mask") (remove_unused_layers no) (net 27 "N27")))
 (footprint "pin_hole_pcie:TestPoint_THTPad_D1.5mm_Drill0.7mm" (layer "F.Cu") (at 135.75 93.3 180)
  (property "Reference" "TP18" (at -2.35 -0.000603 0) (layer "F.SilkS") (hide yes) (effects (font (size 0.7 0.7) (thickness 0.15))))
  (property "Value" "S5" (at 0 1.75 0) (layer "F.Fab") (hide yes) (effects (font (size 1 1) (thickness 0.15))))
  (pad "1" thru_hole circle (at 0 0 180) (size 1.3 1.5) (drill 1) (layers "*.Cu" "*.Mask") (remove_unused_layers no) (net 17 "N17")))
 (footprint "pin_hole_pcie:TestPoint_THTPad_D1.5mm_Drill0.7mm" (layer "F.Cu") (at 137.75 100.3 180)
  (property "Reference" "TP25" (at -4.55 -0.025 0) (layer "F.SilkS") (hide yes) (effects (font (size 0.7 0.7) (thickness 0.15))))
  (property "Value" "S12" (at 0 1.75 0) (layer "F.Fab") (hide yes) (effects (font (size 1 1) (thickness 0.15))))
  (pad "1" thru_hole circle (at 0 0 180) (size 1.3 1.5) (drill 1) (layers "*.Cu" "*.Mask") (remove_unused_layers no) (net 22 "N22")))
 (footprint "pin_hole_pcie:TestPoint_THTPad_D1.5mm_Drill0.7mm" (layer "F.Cu") (at 137.75 82.3 180)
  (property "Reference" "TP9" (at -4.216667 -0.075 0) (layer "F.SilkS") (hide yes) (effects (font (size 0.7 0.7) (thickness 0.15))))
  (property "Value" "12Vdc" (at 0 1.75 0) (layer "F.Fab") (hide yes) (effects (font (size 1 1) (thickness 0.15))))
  (pad "1" thru_hole circle (at 0 0 180) (size 1.3 1.5) (drill 1) (layers "*.Cu" "*.Mask") (remove_unused_layers no) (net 11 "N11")))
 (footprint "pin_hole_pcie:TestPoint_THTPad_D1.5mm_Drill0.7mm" (layer "F.Cu") (at 135.75 105.3 180)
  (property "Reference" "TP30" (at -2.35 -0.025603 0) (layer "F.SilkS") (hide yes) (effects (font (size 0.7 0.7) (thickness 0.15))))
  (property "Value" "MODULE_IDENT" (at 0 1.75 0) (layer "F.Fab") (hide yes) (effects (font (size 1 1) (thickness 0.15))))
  (pad "1" thru_hole circle (at 0 0 180) (size 1.3 1.5) (drill 1) (layers "*.Cu" "*.Mask") (remove_unused_layers no) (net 25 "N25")))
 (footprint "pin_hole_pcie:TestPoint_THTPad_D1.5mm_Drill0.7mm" (layer "F.Cu") (at 137.75 98.3 180)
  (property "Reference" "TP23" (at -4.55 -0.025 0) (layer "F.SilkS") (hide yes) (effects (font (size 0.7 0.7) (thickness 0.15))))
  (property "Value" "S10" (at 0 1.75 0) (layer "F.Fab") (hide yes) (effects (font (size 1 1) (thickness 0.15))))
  (pad "1" thru_hole circle (at 0 0 180) (size 1.3 1.5) (drill 1) (layers "*.Cu" "*.Mask") (remove_unused_layers no) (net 21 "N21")))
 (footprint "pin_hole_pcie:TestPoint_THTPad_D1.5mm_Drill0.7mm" (layer "F.Cu") (at 135.75 91.3 180)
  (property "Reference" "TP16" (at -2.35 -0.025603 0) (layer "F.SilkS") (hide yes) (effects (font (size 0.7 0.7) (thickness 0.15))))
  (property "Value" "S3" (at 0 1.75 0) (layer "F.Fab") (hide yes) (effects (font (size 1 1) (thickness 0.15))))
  (pad "1" thru_hole circle (at 0 0 180) (size 1.3 1.5) (drill 1) (layers "*.Cu" "*.Mask") (remove_unused_layers no) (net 15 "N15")))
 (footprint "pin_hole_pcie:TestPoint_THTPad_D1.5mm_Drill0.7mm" (layer "F.Cu") (at 137.75 76.3 180)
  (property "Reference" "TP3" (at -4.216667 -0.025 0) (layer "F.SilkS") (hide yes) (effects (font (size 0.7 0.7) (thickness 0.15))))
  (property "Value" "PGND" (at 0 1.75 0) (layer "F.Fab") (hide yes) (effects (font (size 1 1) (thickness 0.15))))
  (pad "1" thru_hole circle (at 0 0 180) (size 1.3 1.5) (drill 1) (layers "*.Cu" "*.Mask") (remove_unused_layers no) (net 4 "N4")))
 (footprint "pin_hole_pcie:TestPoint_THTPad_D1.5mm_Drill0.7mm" (layer "F.Cu") (at 137.75 92.3 180)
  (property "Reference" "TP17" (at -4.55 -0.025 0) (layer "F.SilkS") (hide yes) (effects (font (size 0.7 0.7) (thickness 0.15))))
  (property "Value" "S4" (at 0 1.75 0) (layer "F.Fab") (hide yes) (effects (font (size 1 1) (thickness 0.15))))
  (pad "1" thru_hole circle (at 0 0 180) (size 1.3 1.5) (drill 1) (layers "*.Cu" "*.Mask") (remove_unused_layers no) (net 16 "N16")))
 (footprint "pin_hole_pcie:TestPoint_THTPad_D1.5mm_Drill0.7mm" (layer "F.Cu") (at 137.75 106.3 180)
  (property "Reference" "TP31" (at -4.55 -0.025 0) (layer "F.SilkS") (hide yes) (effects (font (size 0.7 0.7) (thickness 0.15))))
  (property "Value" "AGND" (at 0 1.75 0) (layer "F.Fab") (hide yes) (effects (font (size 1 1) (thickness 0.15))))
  (pad "1" thru_hole circle (at 0 0 180) (size 1.3 1.5) (drill 1) (layers "*.Cu" "*.Mask") (remove_unused_layers no) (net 26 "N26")))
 (gr_rect (start 134.78 71.21) (end 148.22 110.47) (stroke (width 0.05) (type default)) (fill no) (layer "Edge.Cuts"))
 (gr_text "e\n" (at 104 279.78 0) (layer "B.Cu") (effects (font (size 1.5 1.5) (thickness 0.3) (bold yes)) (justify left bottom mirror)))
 (segment (start 137.75 74.3) (end 145.3 74.3) (width 0.2) (layer "B.Cu") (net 1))
 (segment (start 140.8 75.3) (end 147.3 75.3) (width 0.2) (layer "B.Cu") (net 4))
 (segment (start 137.75 78.3) (end 145.3 78.3) (width 0.2) (layer "B.Cu") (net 4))
 (segment (start 135.75 75.3) (end 140.8 75.3) (width 0.2) (layer "B.Cu") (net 4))
 (segment (start 135.75 77.3) (end 147.3 77.3) (width 0.2) (layer "B.Cu") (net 4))
 (segment (start 137.75 76.3) (end 145.3 76.3) (width 0.2) (layer "B.Cu") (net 4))
 (segment (start 135.75 79.3) (end 147.3 79.3) (width 0.2) (layer "B.Cu") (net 10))
 (segment (start 135.75 81.3) (end 147.3 81.3) (width 0.2) (layer "B.Cu") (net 11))
 (segment (start 137.75 82.3) (end 145.3 82.3) (width 0.2) (layer "B.Cu") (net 11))
 (segment (start 137.75 80.3) (end 145.3 80.3) (width 0.2) (layer "B.Cu") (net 11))
 (segment (start 140.17 83.3) (end 140.8 83.3) (width 0.3) (layer "B.Cu") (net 12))
 (segment (start 136.83 83.94) (end 137.13 83.64) (width 0.3) (layer "B.Cu") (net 12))
 (segment (start 135.75 83.94) (end 136.83 83.94) (width 0.3) (layer "B.Cu") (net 12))
 (segment (start 139.83 83.64) (end 140.17 83.3) (width 0.3) (layer "B.Cu") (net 12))
 (segment (start 137.13 83.64) (end 139.83 83.64) (width 0.3) (layer "B.Cu") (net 12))
 (segment (start 140.8 83.3) (end 147.3 83.3) (width 0.3) (layer "B.Cu") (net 12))
 (segment (start 142.8 84.3) (end 145.3 84.3) (width 0.3) (layer "B.Cu") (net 7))
 (segment (start 141.43 84.94) (end 142.07 84.3) (width 0.3) (layer "B.Cu") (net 7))
 (segment (start 137.75 84.94) (end 141.43 84.94) (width 0.3) (layer "B.Cu") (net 7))
 (segment (start 142.07 84.3) (end 142.8 84.3) (width 0.3) (layer "B.Cu") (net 7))
 (segment (start 145.37 87.3) (end 145.18 87.49) (width 0.2) (layer "B.Cu") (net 3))
 (segment (start 142.58 87.49) (end 142.39 87.3) (width 0.2) (layer "B.Cu") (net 3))
 (segment (start 147.3 87.3) (end 145.37 87.3) (width 0.2) (layer "B.Cu") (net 3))
 (segment (start 145.18 87.49) (end 142.58 87.49) (width 0.2) (layer "B.Cu") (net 3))
 (segment (start 135.75 87.3) (end 140.8 87.3) (width 0.2) (layer "B.Cu") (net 3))
 (segment (start 142.39 87.3) (end 140.8 87.3) (width 0.2) (layer "B.Cu") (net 3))
 (segment (start 137.75 88.3) (end 145.3 88.3) (width 0.2) (layer "B.Cu") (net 5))
 (segment (start 140.8 89.3) (end 147.3 89.3) (width 0.2) (layer "B.Cu") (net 13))
 (segment (start 135.75 89.3) (end 140.8 89.3) (width 0.2) (layer "B.Cu") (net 13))
 (segment (start 137.75 90.3) (end 145.3 90.3) (width 0.2) (layer "B.Cu") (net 14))
 (segment (start 135.75 91.3) (end 147.3 91.3) (width 0.2) (layer "B.Cu") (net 15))
 (segment (start 137.75 92.3) (end 145.3 92.3) (width 0.2) (layer "B.Cu") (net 16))
 (segment (start 135.75 93.3) (end 147.3 93.3) (width 0.2) (layer "B.Cu") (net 17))
 (segment (start 137.75 94.3) (end 145.3 94.3) (width 0.2) (layer "B.Cu") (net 2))
 (segment (start 135.75 95.3) (end 147.3 95.3) (width 0.2) (layer "B.Cu") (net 18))
 (segment (start 137.75 96.3) (end 145.3 96.3) (width 0.2) (layer "B.Cu") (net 19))
 (segment (start 135.75 97.3) (end 147.3 97.3) (width 0.2) (layer "B.Cu") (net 20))
 (segment (start 137.75 98.3) (end 145.3 98.3) (width 0.2) (layer "B.Cu") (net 21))
 (segment (start 135.75 99.3) (end 147.3 99.3) (width 0.2) (layer "B.Cu") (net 6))
 (segment (start 137.75 100.3) (end 145.3 100.3) (width 0.2) (layer "B.Cu") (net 22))
 (segment (start 135.75 101.3) (end 147.3 101.3) (width 0.2) (layer "B.Cu") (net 8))
 (segment (start 137.75 102.3) (end 145.3 102.3) (width 0.2) (layer "B.Cu") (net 9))
 (segment (start 135.75 103.3) (end 147.3 103.3) (width 0.2) (layer "B.Cu") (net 23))
 (segment (start 137.75 104.3) (end 145.3 104.3) (width 0.2) (layer "B.Cu") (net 24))
 (segment (start 135.75 105.3) (end 147.3 105.3) (width 0.2) (layer "B.Cu") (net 25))
 (segment (start 137.75 106.3) (end 145.3 106.3) (width 0.2) (layer "B.Cu") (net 26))
 (segment (start 135.75 107.3) (end 147.3 107.3) (width 0.2) (layer "B.Cu") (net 27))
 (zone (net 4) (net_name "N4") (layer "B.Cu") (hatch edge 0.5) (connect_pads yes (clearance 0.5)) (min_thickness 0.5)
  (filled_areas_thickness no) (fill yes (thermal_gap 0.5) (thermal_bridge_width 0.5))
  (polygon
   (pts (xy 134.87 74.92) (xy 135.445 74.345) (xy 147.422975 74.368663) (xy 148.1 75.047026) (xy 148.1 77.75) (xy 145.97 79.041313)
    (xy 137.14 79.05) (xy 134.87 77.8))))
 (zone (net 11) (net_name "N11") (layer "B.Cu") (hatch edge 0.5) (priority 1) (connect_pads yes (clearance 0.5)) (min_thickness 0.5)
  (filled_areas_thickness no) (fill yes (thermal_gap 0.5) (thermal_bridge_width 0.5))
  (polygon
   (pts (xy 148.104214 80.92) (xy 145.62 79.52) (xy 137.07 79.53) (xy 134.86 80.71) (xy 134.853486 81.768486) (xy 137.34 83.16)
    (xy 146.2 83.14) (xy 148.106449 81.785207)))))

